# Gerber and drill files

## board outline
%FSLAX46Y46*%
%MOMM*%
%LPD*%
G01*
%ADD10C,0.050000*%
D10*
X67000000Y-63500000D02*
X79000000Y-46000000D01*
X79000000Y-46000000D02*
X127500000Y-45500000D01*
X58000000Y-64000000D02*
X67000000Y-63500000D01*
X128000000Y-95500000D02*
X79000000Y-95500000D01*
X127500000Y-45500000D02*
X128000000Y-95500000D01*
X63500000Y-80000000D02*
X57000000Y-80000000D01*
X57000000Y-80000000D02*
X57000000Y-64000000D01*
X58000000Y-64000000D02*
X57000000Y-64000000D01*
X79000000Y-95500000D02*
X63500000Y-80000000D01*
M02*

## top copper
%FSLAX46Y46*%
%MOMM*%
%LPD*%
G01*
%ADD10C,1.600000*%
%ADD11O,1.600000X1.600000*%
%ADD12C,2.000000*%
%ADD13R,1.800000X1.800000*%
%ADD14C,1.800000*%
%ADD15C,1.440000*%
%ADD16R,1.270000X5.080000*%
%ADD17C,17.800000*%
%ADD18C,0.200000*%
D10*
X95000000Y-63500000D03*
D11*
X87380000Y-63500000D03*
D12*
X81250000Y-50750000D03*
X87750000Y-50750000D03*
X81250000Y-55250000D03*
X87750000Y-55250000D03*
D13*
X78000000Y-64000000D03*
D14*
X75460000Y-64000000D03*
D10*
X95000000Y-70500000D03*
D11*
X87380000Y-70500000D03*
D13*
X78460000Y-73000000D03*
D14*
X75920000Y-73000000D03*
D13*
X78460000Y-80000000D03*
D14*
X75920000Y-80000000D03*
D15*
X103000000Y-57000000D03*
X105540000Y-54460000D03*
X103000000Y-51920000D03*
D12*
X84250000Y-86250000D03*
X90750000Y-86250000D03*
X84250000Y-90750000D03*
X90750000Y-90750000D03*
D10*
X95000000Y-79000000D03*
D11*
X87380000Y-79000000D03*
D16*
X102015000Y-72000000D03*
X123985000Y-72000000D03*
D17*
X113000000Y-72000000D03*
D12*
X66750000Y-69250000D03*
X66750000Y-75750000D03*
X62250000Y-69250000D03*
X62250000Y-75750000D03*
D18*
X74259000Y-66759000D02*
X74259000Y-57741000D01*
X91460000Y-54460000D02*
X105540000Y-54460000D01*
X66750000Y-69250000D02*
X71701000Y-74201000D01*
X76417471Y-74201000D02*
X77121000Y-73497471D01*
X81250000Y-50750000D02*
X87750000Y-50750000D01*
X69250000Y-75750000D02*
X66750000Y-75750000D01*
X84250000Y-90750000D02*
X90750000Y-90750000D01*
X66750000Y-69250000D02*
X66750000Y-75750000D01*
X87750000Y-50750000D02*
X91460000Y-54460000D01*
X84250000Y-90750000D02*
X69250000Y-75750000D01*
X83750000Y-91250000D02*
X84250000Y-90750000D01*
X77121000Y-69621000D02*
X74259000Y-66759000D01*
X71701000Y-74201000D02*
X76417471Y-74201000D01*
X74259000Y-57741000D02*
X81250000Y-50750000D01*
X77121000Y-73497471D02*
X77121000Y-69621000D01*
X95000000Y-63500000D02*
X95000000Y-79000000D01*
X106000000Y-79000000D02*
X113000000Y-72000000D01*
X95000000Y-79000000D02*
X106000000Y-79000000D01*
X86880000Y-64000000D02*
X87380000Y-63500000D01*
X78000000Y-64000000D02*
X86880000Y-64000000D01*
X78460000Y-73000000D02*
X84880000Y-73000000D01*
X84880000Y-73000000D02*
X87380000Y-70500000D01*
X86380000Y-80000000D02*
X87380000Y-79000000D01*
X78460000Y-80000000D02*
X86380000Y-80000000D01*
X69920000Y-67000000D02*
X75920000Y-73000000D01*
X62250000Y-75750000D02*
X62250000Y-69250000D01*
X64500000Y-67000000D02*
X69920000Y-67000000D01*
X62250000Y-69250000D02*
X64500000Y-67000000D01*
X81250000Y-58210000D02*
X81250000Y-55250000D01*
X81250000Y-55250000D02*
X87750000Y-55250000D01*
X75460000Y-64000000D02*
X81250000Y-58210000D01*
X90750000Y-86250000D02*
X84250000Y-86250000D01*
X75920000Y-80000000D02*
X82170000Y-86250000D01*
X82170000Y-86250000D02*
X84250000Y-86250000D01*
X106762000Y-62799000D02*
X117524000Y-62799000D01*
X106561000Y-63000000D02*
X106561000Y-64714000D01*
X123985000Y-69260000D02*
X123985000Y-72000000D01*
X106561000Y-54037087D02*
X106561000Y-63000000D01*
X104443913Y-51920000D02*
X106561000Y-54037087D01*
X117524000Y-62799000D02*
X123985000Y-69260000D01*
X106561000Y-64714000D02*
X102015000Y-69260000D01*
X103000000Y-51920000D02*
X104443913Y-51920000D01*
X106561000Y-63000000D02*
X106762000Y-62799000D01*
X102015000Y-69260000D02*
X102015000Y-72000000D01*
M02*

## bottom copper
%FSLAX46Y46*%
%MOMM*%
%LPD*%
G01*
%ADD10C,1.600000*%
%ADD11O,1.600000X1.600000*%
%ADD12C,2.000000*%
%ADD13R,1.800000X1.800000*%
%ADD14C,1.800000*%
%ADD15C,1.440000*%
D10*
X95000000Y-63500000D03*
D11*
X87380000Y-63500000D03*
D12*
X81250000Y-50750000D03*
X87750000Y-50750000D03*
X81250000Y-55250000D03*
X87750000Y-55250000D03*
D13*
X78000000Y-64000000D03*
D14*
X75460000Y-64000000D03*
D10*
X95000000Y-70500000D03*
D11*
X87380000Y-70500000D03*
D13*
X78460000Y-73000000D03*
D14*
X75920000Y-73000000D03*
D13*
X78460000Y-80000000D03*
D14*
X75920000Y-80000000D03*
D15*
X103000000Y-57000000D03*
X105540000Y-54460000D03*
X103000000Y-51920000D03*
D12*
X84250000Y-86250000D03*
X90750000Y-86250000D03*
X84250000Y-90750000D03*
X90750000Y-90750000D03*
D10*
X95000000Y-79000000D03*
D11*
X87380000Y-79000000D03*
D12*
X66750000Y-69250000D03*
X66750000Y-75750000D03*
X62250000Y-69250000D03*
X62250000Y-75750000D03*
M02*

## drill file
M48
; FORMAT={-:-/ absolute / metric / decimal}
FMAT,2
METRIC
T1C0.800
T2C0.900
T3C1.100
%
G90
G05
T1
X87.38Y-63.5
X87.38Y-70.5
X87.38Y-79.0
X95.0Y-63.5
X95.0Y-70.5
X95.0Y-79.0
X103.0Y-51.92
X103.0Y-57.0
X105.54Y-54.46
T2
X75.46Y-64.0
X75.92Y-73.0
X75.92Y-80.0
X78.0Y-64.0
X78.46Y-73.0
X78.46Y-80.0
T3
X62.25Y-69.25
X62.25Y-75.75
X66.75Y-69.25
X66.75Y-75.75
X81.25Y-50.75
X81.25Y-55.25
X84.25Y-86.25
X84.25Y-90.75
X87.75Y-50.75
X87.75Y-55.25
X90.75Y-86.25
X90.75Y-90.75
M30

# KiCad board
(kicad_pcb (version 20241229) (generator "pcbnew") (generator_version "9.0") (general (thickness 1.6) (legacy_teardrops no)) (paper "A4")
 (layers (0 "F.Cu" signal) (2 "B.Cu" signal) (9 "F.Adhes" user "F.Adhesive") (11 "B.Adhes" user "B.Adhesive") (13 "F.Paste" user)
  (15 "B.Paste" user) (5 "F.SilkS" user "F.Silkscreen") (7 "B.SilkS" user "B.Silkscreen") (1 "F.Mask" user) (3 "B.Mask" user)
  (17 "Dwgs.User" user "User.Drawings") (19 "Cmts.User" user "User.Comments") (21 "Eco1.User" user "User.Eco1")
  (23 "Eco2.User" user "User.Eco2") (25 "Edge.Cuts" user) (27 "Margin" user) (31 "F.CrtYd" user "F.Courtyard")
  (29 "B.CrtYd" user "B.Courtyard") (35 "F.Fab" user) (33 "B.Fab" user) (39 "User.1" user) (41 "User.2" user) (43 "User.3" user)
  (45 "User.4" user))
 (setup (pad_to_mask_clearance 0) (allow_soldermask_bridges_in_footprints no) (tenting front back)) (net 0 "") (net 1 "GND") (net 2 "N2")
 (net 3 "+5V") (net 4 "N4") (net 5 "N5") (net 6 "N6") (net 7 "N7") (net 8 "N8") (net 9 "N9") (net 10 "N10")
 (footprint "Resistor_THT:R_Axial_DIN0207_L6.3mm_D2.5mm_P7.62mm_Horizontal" (layer "F.Cu") (at 95 63.5 180)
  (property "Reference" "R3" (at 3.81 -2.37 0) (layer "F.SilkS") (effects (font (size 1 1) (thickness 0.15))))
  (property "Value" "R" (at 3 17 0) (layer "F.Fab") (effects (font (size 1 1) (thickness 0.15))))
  (pad "1" thru_hole circle (at 0 0 180) (size 1.6 1.6) (drill 0.8) (layers "*.Cu" "*.Mask") (remove_unused_layers no) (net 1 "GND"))
  (pad "2" thru_hole oval (at 7.62 0 180) (size 1.6 1.6) (drill 0.8) (layers "*.Cu" "*.Mask") (remove_unused_layers no) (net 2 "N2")))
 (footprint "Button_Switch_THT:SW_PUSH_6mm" (layer "F.Cu") (at 81.25 50.75)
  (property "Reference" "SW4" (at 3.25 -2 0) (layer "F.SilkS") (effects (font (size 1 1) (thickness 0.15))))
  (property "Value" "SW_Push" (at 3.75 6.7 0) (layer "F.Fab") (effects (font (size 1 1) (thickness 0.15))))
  (pad "1" thru_hole circle (at 0 0 90) (size 2 2) (drill 1.1) (layers "*.Cu" "*.Mask") (remove_unused_layers no) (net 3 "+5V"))
  (pad "1" thru_hole circle (at 6.5 0 90) (size 2 2) (drill 1.1) (layers "*.Cu" "*.Mask") (remove_unused_layers no) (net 3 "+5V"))
  (pad "2" thru_hole circle (at 0 4.5 90) (size 2 2) (drill 1.1) (layers "*.Cu" "*.Mask") (remove_unused_layers no) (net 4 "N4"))
  (pad "2" thru_hole circle (at 6.5 4.5 90) (size 2 2) (drill 1.1) (layers "*.Cu" "*.Mask") (remove_unused_layers no) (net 4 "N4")))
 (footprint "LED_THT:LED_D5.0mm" (layer "F.Cu") (at 78 64 180)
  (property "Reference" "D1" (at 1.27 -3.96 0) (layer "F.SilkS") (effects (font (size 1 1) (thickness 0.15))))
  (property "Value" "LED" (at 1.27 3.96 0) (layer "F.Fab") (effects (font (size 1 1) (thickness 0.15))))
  (pad "1" thru_hole rect (at 0 0 180) (size 1.8 1.8) (drill 0.9) (layers "*.Cu" "*.Mask") (remove_unused_layers no) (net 2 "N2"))
  (pad "2" thru_hole circle (at 2.54 0 180) (size 1.8 1.8) (drill 0.9) (layers "*.Cu" "*.Mask") (remove_unused_layers no) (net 4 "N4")))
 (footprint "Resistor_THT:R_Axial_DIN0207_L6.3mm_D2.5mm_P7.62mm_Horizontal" (layer "F.Cu") (at 95 70.5 180)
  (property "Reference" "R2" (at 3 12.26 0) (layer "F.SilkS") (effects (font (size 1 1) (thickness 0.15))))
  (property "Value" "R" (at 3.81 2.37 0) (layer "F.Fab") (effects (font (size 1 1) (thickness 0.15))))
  (pad "1" thru_hole circle (at 0 0 180) (size 1.6 1.6) (drill 0.8) (layers "*.Cu" "*.Mask") (remove_unused_layers no) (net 1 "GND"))
  (pad "2" thru_hole oval (at 7.62 0 180) (size 1.6 1.6) (drill 0.8) (layers "*.Cu" "*.Mask") (remove_unused_layers no) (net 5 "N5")))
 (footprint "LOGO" (layer "F.Cu") (at 116.5 52)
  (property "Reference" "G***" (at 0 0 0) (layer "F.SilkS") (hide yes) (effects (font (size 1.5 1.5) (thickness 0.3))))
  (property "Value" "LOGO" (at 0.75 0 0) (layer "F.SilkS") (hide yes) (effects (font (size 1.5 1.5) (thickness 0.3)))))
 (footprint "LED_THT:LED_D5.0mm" (layer "F.Cu") (at 78.46 73 180)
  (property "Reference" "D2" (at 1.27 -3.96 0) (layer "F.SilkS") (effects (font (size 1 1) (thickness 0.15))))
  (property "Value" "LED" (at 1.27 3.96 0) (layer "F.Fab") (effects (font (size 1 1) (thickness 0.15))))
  (pad "1" thru_hole rect (at 0 0 180) (size 1.8 1.8) (drill 0.9) (layers "*.Cu" "*.Mask") (remove_unused_layers no) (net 5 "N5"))
  (pad "2" thru_hole circle (at 2.54 0 180) (size 1.8 1.8) (drill 0.9) (layers "*.Cu" "*.Mask") (remove_unused_layers no) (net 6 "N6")))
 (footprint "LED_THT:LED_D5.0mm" (layer "F.Cu") (at 78.46 80 180)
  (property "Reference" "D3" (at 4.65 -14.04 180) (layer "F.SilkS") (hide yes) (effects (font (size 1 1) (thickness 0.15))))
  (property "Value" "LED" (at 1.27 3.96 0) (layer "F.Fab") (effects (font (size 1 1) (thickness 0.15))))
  (pad "1" thru_hole rect (at 0 0 180) (size 1.8 1.8) (drill 0.9) (layers "*.Cu" "*.Mask") (remove_unused_layers no) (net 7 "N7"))
  (pad "2" thru_hole circle (at 2.54 0 180) (size 1.8 1.8) (drill 0.9) (layers "*.Cu" "*.Mask") (remove_unused_layers no) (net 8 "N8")))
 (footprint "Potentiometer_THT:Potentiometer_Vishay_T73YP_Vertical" (layer "F.Cu") (at 103 57)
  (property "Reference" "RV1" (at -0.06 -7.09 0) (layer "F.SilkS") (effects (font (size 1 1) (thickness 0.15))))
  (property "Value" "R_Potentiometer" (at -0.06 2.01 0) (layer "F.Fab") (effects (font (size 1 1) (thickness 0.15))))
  (pad "1" thru_hole circle (at 0 0) (size 1.44 1.44) (drill 0.8) (layers "*.Cu" "*.Mask") (remove_unused_layers no) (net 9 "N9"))
  (pad "2" thru_hole circle (at 2.54 -2.54) (size 1.44 1.44) (drill 0.8) (layers "*.Cu" "*.Mask") (remove_unused_layers no) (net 3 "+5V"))
  (pad "3" thru_hole circle (at 0 -5.08) (size 1.44 1.44) (drill 0.8) (layers "*.Cu" "*.Mask") (remove_unused_layers no) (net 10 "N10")))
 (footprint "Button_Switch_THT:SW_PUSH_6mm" (layer "F.Cu") (at 84.25 86.25)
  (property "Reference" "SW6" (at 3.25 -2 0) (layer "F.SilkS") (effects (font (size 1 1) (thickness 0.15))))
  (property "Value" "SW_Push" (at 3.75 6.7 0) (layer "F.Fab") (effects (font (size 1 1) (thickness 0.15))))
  (pad "1" thru_hole circle (at 0 0 90) (size 2 2) (drill 1.1) (layers "*.Cu" "*.Mask") (remove_unused_layers no) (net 8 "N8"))
  (pad "1" thru_hole circle (at 6.5 0 90) (size 2 2) (drill 1.1) (layers "*.Cu" "*.Mask") (remove_unused_layers no) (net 8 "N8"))
  (pad "2" thru_hole circle (at 0 4.5 90) (size 2 2) (drill 1.1) (layers "*.Cu" "*.Mask") (remove_unused_layers no) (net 3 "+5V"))
  (pad "2" thru_hole circle (at 6.5 4.5 90) (size 2 2) (drill 1.1) (layers "*.Cu" "*.Mask") (remove_unused_layers no) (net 3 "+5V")))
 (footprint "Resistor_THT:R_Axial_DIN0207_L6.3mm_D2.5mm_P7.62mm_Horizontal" (layer "F.Cu") (at 95 79 180)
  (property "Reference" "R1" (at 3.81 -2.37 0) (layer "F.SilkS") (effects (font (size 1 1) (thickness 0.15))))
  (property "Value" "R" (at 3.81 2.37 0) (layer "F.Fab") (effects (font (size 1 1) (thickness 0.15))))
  (pad "1" thru_hole circle (at 0 0 180) (size 1.6 1.6) (drill 0.8) (layers "*.Cu" "*.Mask") (remove_unused_layers no) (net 1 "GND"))
  (pad "2" thru_hole oval (at 7.62 0 180) (size 1.6 1.6) (drill 0.8) (layers "*.Cu" "*.Mask") (remove_unused_layers no) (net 7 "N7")))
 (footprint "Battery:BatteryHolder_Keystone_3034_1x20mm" (layer "F.Cu") (at 113 72)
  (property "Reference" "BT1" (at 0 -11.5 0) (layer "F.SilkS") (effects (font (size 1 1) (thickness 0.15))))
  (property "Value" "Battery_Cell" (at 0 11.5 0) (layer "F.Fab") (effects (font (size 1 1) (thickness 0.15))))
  (pad "1" smd rect (at -10.985 0) (size 1.27 5.08) (layers "F.Cu" "F.Mask" "F.Paste") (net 10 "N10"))
  (pad "1" smd rect (at 10.985 0) (size 1.27 5.08) (layers "F.Cu" "F.Mask" "F.Paste") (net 10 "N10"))
  (pad "2" smd circle (at 0 0) (size 17.8 17.8) (layers "F.Cu" "F.Mask") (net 1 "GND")))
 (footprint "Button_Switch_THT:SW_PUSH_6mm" (layer "F.Cu") (at 66.75 69.25 -90)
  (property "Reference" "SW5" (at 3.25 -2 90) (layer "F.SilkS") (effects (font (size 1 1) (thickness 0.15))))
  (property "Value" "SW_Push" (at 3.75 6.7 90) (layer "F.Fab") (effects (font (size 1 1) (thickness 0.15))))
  (pad "1" thru_hole circle (at 0 0) (size 2 2) (drill 1.1) (layers "*.Cu" "*.Mask") (remove_unused_layers no) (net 3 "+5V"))
  (pad "1" thru_hole circle (at 6.5 0) (size 2 2) (drill 1.1) (layers "*.Cu" "*.Mask") (remove_unused_layers no) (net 3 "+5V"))
  (pad "2" thru_hole circle (at 0 4.5) (size 2 2) (drill 1.1) (layers "*.Cu" "*.Mask") (remove_unused_layers no) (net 6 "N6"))
  (pad "2" thru_hole circle (at 6.5 4.5) (size 2 2) (drill 1.1) (layers "*.Cu" "*.Mask") (remove_unused_layers no) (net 6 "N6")))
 (gr_line (start 67 63.5) (end 79 46) (stroke (width 0.05) (type default)) (layer "Edge.Cuts"))
 (gr_line (start 79 46) (end 127.5 45.5) (stroke (width 0.05) (type default)) (layer "Edge.Cuts"))
 (gr_line (start 58 64) (end 67 63.5) (stroke (width 0.05) (type default)) (layer "Edge.Cuts"))
 (gr_line (start 128 95.5) (end 79 95.5) (stroke (width 0.05) (type default)) (layer "Edge.Cuts"))
 (gr_line (start 127.5 45.5) (end 128 95.5) (stroke (width 0.05) (type default)) (layer "Edge.Cuts"))
 (gr_line (start 63.5 80) (end 57 80) (stroke (width 0.05) (type default)) (layer "Edge.Cuts"))
 (gr_line (start 57 80) (end 57 64) (stroke (width 0.05) (type default)) (layer "Edge.Cuts"))
 (gr_line (start 58 64) (end 57 64) (stroke (width 0.05) (type default)) (layer "Edge.Cuts"))
 (gr_line (start 79 95.5) (end 63.5 80) (stroke (width 0.05) (type default)) (layer "Edge.Cuts"))
 (segment (start 74.259 66.759) (end 74.259 57.741) (width 0.2) (layer "F.Cu") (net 3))
 (segment (start 91.46 54.46) (end 105.54 54.46) (width 0.2) (layer "F.Cu") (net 3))
 (segment (start 66.75 69.25) (end 71.701 74.201) (width 0.2) (layer "F.Cu") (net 3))
 (segment (start 76.417471 74.201) (end 77.121 73.497471) (width 0.2) (layer "F.Cu") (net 3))
 (segment (start 81.25 50.75) (end 87.75 50.75) (width 0.2) (layer "F.Cu") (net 3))
 (segment (start 69.25 75.75) (end 66.75 75.75) (width 0.2) (layer "F.Cu") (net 3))
 (segment (start 84.25 90.75) (end 90.75 90.75) (width 0.2) (layer "F.Cu") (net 3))
 (segment (start 66.75 69.25) (end 66.75 75.75) (width 0.2) (layer "F.Cu") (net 3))
 (segment (start 87.75 50.75) (end 91.46 54.46) (width 0.2) (layer "F.Cu") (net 3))
 (segment (start 84.25 90.75) (end 69.25 75.75) (width 0.2) (layer "F.Cu") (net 3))
 (segment (start 83.75 91.25) (end 84.25 90.75) (width 0.2) (layer "F.Cu") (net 3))
 (segment (start 77.121 69.621) (end 74.259 66.759) (width 0.2) (layer "F.Cu") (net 3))
 (segment (start 71.701 74.201) (end 76.417471 74.201) (width 0.2) (layer "F.Cu") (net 3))
 (segment (start 74.259 57.741) (end 81.25 50.75) (width 0.2) (layer "F.Cu") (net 3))
 (segment (start 77.121 73.497471) (end 77.121 69.621) (width 0.2) (layer "F.Cu") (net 3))
 (segment (start 95 63.5) (end 95 79) (width 0.2) (layer "F.Cu") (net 1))
 (segment (start 106 79) (end 113 72) (width 0.2) (layer "F.Cu") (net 1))
 (segment (start 95 79) (end 106 79) (width 0.2) (layer "F.Cu") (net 1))
 (segment (start 86.88 64) (end 87.38 63.5) (width 0.2) (layer "F.Cu") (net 2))
 (segment (start 78 64) (end 86.88 64) (width 0.2) (layer "F.Cu") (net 2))
 (segment (start 78.46 73) (end 84.88 73) (width 0.2) (layer "F.Cu") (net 5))
 (segment (start 84.88 73) (end 87.38 70.5) (width 0.2) (layer "F.Cu") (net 5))
 (segment (start 86.38 80) (end 87.38 79) (width 0.2) (layer "F.Cu") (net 7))
 (segment (start 78.46 80) (end 86.38 80) (width 0.2) (layer "F.Cu") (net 7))
 (segment (start 69.92 67) (end 75.92 73) (width 0.2) (layer "F.Cu") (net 6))
 (segment (start 62.25 75.75) (end 62.25 69.25) (width 0.2) (layer "F.Cu") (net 6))
 (segment (start 64.5 67) (end 69.92 67) (width 0.2) (layer "F.Cu") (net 6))
 (segment (start 62.25 69.25) (end 64.5 67) (width 0.2) (layer "F.Cu") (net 6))
 (segment (start 81.25 58.21) (end 81.25 55.25) (width 0.2) (layer "F.Cu") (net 4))
 (segment (start 81.25 55.25) (end 87.75 55.25) (width 0.2) (layer "F.Cu") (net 4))
 (segment (start 75.46 64) (end 81.25 58.21) (width 0.2) (layer "F.Cu") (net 4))
 (segment (start 90.75 86.25) (end 84.25 86.25) (width 0.2) (layer "F.Cu") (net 8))
 (segment (start 75.92 80) (end 82.17 86.25) (width 0.2) (layer "F.Cu") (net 8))
 (segment (start 82.17 86.25) (end 84.25 86.25) (width 0.2) (layer "F.Cu") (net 8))
 (segment (start 106.762 62.799) (end 117.524 62.799) (width 0.2) (layer "F.Cu") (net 10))
 (segment (start 106.561 63) (end 106.561 64.714) (width 0.2) (layer "F.Cu") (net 10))
 (segment (start 123.985 69.26) (end 123.985 72) (width 0.2) (layer "F.Cu") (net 10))
 (segment (start 106.561 54.037087) (end 106.561 63) (width 0.2) (layer "F.Cu") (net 10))
 (segment (start 104.443913 51.92) (end 106.561 54.037087) (width 0.2) (layer "F.Cu") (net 10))
 (segment (start 117.524 62.799) (end 123.985 69.26) (width 0.2) (layer "F.Cu") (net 10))
 (segment (start 106.561 64.714) (end 102.015 69.26) (width 0.2) (layer "F.Cu") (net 10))
 (segment (start 103 51.92) (end 104.443913 51.92) (width 0.2) (layer "F.Cu") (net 10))
 (segment (start 106.561 63) (end 106.762 62.799) (width 0.2) (layer "F.Cu") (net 10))
 (segment (start 102.015 69.26) (end 102.015 72) (width 0.2) (layer "F.Cu") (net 10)))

